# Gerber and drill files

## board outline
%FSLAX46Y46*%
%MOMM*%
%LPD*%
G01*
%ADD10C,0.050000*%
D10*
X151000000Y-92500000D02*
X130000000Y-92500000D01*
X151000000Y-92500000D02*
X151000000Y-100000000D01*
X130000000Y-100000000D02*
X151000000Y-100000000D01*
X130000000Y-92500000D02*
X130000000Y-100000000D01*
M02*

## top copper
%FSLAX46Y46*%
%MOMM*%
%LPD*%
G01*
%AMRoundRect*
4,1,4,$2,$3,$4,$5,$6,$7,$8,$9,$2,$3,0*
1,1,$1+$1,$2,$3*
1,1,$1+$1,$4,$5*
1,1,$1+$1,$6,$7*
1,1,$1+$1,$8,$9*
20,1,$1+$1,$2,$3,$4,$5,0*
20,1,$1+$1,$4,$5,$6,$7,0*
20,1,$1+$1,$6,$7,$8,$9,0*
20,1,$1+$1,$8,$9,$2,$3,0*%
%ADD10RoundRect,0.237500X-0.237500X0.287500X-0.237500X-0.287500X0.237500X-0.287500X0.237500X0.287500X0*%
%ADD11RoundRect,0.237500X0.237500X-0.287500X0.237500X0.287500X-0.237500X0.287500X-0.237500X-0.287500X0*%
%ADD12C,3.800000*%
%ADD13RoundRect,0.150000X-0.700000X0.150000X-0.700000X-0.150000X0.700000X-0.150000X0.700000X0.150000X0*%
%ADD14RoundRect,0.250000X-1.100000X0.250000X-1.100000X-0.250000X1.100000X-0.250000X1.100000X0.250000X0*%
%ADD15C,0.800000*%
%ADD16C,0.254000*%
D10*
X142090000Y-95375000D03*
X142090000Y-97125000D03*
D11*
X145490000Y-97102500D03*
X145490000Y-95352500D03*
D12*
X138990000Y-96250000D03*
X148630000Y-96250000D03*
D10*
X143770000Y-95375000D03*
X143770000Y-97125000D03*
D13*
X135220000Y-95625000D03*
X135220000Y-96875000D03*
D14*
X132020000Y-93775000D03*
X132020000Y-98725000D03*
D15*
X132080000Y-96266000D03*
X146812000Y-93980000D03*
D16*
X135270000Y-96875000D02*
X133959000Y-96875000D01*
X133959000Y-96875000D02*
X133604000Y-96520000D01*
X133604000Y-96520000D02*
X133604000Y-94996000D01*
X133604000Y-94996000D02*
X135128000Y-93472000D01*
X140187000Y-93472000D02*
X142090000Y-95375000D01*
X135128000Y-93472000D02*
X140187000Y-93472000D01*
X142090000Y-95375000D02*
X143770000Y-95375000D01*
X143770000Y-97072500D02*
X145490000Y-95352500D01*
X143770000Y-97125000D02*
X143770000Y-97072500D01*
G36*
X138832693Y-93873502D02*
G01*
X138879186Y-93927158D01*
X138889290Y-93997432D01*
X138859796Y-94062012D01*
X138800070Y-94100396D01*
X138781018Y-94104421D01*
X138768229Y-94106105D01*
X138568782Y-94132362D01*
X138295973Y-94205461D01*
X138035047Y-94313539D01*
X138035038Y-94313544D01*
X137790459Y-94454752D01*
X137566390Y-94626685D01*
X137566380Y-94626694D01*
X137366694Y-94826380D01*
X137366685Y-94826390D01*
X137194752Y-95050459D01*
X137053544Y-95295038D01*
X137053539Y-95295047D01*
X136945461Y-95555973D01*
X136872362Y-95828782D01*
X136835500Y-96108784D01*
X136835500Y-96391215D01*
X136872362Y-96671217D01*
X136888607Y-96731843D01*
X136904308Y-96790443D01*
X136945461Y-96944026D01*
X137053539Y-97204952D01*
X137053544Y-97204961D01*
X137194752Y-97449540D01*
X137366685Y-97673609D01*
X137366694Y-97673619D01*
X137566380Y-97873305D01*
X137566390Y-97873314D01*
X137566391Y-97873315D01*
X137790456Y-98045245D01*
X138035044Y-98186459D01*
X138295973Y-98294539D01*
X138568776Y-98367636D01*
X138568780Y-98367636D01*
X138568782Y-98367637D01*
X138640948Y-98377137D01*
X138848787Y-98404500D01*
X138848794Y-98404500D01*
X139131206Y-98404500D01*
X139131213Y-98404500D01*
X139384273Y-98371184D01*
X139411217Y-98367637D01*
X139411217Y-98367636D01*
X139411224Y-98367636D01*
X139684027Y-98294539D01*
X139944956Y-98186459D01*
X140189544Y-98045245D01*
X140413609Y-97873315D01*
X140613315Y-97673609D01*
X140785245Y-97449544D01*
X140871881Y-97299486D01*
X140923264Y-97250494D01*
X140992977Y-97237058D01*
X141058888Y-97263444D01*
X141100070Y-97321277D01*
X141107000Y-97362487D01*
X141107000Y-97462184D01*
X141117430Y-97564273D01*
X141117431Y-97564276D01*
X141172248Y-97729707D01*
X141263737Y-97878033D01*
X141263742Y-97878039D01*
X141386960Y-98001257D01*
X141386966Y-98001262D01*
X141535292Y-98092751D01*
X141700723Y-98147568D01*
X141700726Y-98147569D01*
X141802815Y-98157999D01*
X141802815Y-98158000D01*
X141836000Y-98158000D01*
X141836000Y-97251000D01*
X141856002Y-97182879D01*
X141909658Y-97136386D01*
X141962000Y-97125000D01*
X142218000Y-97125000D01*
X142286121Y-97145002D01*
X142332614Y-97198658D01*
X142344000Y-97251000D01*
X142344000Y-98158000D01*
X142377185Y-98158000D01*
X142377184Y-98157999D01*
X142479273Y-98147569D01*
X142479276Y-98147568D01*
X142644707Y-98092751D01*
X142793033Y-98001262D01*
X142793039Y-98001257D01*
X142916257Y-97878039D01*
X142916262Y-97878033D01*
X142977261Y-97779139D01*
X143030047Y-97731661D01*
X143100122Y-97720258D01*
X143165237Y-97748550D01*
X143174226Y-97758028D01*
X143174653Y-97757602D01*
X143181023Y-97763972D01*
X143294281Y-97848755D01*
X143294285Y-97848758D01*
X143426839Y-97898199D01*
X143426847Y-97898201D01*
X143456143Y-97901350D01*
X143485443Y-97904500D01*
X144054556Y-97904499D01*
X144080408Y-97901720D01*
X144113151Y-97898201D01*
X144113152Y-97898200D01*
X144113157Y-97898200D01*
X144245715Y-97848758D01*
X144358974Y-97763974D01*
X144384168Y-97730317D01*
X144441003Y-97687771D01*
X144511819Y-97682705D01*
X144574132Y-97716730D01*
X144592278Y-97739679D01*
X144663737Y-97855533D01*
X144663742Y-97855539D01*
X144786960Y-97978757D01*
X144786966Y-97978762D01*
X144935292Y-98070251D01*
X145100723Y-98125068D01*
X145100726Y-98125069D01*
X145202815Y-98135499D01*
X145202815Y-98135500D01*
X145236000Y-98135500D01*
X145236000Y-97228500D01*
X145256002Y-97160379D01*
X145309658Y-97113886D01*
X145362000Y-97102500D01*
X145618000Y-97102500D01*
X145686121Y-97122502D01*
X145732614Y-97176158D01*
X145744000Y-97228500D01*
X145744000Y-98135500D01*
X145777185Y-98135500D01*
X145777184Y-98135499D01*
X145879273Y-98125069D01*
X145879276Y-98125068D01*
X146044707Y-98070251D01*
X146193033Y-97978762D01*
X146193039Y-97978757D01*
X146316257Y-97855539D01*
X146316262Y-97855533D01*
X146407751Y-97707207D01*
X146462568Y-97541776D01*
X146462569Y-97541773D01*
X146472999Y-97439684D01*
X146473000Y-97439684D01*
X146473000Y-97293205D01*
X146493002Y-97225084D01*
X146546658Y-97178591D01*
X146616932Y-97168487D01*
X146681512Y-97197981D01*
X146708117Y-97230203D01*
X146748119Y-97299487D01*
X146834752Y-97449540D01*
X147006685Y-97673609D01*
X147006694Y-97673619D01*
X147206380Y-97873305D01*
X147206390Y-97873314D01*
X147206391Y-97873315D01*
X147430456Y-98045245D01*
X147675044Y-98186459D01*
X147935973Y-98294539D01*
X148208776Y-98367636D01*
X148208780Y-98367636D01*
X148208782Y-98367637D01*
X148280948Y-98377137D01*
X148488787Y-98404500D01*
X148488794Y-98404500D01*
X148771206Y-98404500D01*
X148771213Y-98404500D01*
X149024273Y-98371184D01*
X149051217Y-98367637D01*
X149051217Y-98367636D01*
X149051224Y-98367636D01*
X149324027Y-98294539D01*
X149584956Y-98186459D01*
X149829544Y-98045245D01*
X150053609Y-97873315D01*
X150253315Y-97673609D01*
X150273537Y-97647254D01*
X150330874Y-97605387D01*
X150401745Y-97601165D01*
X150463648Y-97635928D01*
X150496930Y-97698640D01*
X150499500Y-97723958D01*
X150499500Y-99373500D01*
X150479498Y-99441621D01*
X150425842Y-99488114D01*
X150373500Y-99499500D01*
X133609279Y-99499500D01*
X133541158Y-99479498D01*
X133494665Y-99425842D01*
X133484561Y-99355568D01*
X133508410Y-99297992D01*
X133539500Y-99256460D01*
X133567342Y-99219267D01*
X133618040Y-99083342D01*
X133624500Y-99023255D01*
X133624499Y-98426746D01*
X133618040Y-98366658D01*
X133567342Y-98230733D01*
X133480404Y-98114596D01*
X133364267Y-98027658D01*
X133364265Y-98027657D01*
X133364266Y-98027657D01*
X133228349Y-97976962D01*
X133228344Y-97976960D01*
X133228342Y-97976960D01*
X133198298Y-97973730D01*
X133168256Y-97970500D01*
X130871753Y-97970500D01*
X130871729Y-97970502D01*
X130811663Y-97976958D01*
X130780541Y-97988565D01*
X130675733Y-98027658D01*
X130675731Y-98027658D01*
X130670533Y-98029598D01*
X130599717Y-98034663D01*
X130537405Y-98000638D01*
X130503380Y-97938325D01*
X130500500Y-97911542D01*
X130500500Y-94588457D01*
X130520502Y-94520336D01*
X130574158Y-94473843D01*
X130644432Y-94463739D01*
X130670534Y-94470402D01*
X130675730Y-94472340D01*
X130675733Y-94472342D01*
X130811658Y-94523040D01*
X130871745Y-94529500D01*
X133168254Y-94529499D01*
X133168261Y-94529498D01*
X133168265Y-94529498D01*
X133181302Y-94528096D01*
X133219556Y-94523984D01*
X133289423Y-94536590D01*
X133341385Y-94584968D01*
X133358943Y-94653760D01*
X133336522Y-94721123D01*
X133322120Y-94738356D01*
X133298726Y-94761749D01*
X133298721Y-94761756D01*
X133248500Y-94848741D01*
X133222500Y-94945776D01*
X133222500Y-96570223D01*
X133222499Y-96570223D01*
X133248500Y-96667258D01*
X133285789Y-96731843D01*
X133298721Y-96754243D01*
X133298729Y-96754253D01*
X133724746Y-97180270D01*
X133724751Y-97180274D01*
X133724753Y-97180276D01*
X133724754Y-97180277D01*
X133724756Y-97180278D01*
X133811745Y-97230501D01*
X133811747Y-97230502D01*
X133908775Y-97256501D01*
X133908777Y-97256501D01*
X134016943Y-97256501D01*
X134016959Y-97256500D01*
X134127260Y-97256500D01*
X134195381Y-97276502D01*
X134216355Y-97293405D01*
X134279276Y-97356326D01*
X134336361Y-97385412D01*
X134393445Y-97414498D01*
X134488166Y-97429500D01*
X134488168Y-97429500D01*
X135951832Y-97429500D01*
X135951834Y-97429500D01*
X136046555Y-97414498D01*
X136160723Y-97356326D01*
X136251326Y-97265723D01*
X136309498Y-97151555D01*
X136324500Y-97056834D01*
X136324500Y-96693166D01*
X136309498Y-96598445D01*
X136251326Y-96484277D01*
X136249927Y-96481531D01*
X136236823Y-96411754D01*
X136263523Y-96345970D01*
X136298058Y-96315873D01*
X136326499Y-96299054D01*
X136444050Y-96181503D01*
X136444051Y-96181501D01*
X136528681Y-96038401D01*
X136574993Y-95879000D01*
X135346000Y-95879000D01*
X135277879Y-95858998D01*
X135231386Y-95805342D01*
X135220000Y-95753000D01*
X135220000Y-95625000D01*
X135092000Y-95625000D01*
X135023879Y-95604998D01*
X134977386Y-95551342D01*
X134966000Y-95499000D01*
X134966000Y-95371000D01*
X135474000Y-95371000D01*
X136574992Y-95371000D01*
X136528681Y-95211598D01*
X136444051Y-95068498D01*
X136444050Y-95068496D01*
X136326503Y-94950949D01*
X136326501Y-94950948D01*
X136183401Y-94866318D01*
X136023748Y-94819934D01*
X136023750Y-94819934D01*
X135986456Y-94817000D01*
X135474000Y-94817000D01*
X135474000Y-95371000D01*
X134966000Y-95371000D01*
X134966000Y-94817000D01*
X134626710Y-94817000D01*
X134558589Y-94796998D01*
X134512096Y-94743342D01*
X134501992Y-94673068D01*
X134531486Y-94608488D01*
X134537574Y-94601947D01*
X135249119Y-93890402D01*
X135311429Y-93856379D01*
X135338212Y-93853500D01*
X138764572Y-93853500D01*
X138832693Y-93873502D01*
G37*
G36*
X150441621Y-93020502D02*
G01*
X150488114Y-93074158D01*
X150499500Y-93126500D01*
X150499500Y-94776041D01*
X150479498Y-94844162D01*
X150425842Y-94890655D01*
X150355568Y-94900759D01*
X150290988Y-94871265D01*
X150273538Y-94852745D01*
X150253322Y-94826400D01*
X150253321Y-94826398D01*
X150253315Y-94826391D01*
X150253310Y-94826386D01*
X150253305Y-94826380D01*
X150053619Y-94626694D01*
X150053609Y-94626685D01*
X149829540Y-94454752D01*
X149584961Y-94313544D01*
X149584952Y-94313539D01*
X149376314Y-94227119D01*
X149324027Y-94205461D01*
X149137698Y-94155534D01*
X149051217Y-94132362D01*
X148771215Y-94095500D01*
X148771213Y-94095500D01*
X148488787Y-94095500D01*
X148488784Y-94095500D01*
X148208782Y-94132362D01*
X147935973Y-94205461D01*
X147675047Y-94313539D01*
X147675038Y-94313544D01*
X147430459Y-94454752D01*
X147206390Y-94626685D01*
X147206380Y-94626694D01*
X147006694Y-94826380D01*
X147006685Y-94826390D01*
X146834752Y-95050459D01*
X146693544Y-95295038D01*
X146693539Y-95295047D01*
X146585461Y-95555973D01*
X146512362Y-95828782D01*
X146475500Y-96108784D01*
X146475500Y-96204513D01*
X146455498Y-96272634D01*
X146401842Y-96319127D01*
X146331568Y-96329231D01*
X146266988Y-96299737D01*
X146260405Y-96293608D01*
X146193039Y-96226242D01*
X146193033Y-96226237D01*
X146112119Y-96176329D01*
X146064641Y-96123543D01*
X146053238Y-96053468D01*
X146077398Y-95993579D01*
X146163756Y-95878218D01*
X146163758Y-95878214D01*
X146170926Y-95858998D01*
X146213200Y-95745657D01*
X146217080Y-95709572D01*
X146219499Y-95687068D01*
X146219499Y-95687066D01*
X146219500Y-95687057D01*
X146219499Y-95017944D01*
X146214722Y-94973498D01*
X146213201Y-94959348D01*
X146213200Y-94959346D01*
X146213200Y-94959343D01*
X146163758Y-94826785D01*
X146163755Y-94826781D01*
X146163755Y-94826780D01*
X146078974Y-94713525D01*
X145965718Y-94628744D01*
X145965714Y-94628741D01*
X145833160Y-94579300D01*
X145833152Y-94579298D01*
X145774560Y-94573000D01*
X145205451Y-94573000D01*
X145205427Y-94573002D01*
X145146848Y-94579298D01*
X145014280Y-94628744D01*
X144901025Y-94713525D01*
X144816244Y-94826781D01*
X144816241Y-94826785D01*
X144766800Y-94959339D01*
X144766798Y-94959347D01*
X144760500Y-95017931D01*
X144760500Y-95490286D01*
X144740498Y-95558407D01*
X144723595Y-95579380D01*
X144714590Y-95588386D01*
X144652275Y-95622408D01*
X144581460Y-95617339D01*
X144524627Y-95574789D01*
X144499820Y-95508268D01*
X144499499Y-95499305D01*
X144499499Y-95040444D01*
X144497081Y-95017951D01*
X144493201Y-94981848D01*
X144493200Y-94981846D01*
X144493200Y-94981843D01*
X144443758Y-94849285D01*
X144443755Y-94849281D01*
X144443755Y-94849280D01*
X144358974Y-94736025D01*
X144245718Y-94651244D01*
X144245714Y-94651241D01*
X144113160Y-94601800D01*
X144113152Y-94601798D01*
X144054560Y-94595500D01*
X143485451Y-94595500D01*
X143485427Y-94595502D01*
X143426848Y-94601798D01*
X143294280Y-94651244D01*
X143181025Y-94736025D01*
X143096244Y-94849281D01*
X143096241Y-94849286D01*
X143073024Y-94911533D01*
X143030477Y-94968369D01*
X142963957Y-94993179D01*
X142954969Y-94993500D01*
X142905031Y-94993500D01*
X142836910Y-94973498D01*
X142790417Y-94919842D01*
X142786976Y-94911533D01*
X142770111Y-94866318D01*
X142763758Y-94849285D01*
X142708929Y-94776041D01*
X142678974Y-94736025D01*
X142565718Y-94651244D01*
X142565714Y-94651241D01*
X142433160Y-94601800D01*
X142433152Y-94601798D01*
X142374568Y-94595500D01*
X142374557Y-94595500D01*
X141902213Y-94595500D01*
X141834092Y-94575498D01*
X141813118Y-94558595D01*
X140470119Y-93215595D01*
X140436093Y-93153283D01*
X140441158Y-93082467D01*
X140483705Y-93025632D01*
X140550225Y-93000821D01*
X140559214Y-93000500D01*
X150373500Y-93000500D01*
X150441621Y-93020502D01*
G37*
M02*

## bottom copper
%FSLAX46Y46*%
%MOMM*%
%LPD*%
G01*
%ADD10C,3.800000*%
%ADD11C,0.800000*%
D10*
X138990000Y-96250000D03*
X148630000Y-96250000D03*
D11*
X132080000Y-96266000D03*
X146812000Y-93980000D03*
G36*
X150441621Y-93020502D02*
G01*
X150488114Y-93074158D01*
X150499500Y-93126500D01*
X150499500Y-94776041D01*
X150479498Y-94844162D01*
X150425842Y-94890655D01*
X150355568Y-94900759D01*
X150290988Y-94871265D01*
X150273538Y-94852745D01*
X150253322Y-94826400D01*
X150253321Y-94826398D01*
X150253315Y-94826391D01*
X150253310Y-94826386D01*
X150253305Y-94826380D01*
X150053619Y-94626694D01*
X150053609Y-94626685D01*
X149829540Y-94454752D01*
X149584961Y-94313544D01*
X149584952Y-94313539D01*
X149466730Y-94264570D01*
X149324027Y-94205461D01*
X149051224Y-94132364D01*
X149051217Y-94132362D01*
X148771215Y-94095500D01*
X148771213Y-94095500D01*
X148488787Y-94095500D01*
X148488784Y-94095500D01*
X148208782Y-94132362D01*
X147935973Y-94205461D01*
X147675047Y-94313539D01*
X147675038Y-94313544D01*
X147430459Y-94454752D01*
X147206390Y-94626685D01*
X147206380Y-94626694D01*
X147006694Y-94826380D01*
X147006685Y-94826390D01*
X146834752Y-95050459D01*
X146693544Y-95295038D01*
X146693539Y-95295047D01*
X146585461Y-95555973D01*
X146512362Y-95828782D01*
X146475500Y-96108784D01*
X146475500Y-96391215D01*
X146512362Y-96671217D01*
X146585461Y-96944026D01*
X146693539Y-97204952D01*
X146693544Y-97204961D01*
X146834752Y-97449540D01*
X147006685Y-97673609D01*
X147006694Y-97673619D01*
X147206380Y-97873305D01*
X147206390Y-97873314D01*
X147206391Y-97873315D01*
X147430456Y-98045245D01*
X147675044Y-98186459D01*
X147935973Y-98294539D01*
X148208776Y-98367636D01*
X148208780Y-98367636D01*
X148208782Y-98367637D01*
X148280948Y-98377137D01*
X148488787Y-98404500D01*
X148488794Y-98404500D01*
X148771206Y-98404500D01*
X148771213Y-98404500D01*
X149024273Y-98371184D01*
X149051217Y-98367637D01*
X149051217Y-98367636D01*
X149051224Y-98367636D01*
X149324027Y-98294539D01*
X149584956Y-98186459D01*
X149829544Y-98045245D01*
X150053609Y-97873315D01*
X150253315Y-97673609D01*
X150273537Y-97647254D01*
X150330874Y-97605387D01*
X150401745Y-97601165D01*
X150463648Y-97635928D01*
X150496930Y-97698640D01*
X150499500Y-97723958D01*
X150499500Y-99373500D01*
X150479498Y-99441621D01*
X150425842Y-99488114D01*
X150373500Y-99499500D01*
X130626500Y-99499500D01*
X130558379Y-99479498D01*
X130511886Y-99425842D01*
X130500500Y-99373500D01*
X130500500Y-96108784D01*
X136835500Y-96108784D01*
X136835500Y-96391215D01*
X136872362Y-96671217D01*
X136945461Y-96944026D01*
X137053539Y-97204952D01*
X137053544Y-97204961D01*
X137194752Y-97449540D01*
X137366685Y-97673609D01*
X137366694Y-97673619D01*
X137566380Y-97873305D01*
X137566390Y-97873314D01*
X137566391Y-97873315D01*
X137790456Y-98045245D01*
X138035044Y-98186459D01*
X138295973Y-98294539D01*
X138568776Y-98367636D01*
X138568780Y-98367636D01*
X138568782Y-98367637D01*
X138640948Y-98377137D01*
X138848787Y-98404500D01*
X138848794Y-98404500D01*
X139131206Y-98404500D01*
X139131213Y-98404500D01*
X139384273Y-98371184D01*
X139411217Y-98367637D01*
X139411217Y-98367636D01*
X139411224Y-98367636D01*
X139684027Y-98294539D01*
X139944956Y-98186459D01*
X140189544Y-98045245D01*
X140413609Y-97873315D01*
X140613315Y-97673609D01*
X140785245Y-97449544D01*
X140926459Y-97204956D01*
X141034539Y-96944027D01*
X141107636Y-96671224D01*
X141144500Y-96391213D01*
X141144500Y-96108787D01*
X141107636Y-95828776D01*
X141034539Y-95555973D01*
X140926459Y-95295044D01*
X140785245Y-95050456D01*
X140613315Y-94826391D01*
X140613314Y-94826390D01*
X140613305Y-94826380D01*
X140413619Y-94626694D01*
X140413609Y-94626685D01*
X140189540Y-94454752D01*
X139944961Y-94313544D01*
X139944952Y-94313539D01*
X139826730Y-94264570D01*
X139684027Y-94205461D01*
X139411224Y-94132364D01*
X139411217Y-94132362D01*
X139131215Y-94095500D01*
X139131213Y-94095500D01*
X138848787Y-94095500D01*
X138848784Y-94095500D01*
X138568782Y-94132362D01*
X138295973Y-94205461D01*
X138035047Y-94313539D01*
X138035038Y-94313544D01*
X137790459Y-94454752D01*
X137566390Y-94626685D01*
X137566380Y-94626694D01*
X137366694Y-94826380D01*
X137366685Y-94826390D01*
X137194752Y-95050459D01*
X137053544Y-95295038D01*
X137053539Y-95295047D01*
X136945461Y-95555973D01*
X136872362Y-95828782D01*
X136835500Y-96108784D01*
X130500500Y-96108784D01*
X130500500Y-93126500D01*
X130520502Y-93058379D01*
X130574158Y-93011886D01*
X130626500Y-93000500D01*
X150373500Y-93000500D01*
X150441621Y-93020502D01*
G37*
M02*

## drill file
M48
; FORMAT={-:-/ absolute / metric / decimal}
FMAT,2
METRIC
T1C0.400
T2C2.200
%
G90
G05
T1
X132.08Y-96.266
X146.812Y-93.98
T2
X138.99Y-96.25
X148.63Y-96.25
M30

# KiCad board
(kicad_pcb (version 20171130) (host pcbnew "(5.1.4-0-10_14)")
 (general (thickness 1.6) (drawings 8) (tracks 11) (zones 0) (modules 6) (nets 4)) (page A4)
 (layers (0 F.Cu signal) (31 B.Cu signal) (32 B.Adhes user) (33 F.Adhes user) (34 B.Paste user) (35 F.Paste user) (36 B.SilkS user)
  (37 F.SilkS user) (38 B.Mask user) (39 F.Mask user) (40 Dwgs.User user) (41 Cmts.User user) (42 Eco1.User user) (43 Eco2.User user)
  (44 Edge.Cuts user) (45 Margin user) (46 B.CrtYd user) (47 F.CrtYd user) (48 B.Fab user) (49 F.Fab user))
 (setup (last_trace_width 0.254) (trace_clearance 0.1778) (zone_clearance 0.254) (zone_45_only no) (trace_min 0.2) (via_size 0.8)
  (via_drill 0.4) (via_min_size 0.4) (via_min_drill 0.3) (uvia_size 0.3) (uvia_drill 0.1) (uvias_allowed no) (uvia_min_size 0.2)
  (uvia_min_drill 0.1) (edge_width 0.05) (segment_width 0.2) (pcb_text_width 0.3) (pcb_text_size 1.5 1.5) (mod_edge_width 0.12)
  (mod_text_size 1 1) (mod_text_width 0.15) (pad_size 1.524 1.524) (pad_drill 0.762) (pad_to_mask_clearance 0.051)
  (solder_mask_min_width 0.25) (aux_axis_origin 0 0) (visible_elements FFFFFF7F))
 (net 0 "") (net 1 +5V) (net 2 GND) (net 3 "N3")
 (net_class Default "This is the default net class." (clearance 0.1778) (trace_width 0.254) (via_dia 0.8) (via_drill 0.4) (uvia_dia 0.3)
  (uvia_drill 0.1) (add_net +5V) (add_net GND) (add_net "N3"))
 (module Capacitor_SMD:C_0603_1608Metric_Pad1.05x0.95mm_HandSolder (layer F.Cu) (at 142.09 96.25 270)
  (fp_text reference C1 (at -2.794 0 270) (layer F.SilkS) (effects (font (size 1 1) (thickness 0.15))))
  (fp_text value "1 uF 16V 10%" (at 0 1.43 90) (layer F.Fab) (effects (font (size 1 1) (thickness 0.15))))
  (pad 1 smd roundrect (at -0.875 0 270) (size 1.05 0.95) (layers F.Cu F.Paste F.Mask) (roundrect_rratio 0.25) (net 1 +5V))
  (pad 2 smd roundrect (at 0.875 0 270) (size 1.05 0.95) (layers F.Cu F.Paste F.Mask) (roundrect_rratio 0.25) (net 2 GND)))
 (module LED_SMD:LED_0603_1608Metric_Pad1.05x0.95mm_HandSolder (layer F.Cu) (at 145.49 96.2275 90)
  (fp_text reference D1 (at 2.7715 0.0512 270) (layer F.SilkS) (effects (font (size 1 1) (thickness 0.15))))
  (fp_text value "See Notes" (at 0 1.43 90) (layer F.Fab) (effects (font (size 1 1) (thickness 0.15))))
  (pad 1 smd roundrect (at -0.875 0 90) (size 1.05 0.95) (layers F.Cu F.Paste F.Mask) (roundrect_rratio 0.25) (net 2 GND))
  (pad 2 smd roundrect (at 0.875 0 90) (size 1.05 0.95) (layers F.Cu F.Paste F.Mask) (roundrect_rratio 0.25) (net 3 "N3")))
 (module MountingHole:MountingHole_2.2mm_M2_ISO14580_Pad (layer F.Cu) (at 138.99 96.25)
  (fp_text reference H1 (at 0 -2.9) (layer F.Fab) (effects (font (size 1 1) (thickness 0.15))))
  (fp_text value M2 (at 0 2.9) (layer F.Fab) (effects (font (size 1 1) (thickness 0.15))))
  (pad 1 thru_hole circle (at 0 0) (size 3.8 3.8) (drill 2.2) (layers *.Cu *.Mask)))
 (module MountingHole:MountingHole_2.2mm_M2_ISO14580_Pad (layer F.Cu) (at 148.63 96.25)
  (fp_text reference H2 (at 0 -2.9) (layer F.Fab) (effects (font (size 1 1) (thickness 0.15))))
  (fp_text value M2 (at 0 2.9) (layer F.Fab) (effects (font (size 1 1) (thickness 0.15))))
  (pad 1 thru_hole circle (at 0 0) (size 3.8 3.8) (drill 2.2) (layers *.Cu *.Mask)))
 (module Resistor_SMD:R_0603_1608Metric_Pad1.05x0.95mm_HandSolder (layer F.Cu) (at 143.77 96.25 270)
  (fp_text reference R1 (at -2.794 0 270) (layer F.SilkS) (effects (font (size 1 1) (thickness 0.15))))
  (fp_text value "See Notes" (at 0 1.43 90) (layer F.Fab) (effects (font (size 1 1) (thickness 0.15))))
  (pad 1 smd roundrect (at -0.875 0 270) (size 1.05 0.95) (layers F.Cu F.Paste F.Mask) (roundrect_rratio 0.25) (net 1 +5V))
  (pad 2 smd roundrect (at 0.875 0 270) (size 1.05 0.95) (layers F.Cu F.Paste F.Mask) (roundrect_rratio 0.25) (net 3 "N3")))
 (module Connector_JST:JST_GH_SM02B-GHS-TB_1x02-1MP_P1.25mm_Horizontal (layer F.Cu) (at 133.37 96.25 270)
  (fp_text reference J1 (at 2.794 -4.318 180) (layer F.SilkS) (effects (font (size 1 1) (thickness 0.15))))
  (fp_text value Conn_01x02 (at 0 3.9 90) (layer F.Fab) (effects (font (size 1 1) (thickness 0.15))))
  (pad 1 smd roundrect (at -0.625 -1.85 270) (size 0.6 1.7) (layers F.Cu F.Paste F.Mask) (roundrect_rratio 0.25) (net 2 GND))
  (pad 2 smd roundrect (at 0.625 -1.85 270) (size 0.6 1.7) (layers F.Cu F.Paste F.Mask) (roundrect_rratio 0.25) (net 1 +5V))
  (pad MP smd roundrect (at -2.475 1.35 270) (size 1 2.7) (layers F.Cu F.Paste F.Mask) (roundrect_rratio 0.25))
  (pad MP smd roundrect (at 2.475 1.35 270) (size 1 2.7) (layers F.Cu F.Paste F.Mask) (roundrect_rratio 0.25)))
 (gr_line (start 151 92.5) (end 130 92.5) (layer Edge.Cuts) (width 0.05))
 (gr_line (start 151 92.5) (end 151 100) (layer Edge.Cuts) (width 0.05))
 (gr_line (start 130 100) (end 151 100) (layer Edge.Cuts) (width 0.05))
 (gr_line (start 130 92.5) (end 130 100) (layer Edge.Cuts) (width 0.05))
 (segment (start 135.27 96.875) (end 133.959 96.875) (width 0.254) (layer F.Cu) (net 1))
 (segment (start 133.959 96.875) (end 133.604 96.52) (width 0.254) (layer F.Cu) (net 1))
 (segment (start 133.604 96.52) (end 133.604 94.996) (width 0.254) (layer F.Cu) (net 1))
 (segment (start 133.604 94.996) (end 135.128 93.472) (width 0.254) (layer F.Cu) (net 1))
 (segment (start 140.187 93.472) (end 142.09 95.375) (width 0.254) (layer F.Cu) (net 1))
 (segment (start 135.128 93.472) (end 140.187 93.472) (width 0.254) (layer F.Cu) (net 1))
 (segment (start 142.09 95.375) (end 143.77 95.375) (width 0.254) (layer F.Cu) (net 1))
 (via (at 132.08 96.266) (size 0.8) (drill 0.4) (layers F.Cu B.Cu) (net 2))
 (via (at 146.812 93.98) (size 0.8) (drill 0.4) (layers F.Cu B.Cu) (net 2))
 (segment (start 143.77 97.0725) (end 145.49 95.3525) (width 0.254) (layer F.Cu) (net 3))
 (segment (start 143.77 97.125) (end 143.77 97.0725) (width 0.254) (layer F.Cu) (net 3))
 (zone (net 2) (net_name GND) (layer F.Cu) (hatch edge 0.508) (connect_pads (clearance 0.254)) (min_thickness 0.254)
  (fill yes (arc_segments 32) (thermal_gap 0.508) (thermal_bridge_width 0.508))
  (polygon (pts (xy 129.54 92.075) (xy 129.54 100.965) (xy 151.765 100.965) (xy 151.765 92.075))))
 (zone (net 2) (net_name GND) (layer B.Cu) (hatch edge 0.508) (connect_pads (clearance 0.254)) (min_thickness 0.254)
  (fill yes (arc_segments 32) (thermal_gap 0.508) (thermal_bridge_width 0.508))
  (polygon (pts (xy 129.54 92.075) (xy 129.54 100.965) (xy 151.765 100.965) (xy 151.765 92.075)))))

